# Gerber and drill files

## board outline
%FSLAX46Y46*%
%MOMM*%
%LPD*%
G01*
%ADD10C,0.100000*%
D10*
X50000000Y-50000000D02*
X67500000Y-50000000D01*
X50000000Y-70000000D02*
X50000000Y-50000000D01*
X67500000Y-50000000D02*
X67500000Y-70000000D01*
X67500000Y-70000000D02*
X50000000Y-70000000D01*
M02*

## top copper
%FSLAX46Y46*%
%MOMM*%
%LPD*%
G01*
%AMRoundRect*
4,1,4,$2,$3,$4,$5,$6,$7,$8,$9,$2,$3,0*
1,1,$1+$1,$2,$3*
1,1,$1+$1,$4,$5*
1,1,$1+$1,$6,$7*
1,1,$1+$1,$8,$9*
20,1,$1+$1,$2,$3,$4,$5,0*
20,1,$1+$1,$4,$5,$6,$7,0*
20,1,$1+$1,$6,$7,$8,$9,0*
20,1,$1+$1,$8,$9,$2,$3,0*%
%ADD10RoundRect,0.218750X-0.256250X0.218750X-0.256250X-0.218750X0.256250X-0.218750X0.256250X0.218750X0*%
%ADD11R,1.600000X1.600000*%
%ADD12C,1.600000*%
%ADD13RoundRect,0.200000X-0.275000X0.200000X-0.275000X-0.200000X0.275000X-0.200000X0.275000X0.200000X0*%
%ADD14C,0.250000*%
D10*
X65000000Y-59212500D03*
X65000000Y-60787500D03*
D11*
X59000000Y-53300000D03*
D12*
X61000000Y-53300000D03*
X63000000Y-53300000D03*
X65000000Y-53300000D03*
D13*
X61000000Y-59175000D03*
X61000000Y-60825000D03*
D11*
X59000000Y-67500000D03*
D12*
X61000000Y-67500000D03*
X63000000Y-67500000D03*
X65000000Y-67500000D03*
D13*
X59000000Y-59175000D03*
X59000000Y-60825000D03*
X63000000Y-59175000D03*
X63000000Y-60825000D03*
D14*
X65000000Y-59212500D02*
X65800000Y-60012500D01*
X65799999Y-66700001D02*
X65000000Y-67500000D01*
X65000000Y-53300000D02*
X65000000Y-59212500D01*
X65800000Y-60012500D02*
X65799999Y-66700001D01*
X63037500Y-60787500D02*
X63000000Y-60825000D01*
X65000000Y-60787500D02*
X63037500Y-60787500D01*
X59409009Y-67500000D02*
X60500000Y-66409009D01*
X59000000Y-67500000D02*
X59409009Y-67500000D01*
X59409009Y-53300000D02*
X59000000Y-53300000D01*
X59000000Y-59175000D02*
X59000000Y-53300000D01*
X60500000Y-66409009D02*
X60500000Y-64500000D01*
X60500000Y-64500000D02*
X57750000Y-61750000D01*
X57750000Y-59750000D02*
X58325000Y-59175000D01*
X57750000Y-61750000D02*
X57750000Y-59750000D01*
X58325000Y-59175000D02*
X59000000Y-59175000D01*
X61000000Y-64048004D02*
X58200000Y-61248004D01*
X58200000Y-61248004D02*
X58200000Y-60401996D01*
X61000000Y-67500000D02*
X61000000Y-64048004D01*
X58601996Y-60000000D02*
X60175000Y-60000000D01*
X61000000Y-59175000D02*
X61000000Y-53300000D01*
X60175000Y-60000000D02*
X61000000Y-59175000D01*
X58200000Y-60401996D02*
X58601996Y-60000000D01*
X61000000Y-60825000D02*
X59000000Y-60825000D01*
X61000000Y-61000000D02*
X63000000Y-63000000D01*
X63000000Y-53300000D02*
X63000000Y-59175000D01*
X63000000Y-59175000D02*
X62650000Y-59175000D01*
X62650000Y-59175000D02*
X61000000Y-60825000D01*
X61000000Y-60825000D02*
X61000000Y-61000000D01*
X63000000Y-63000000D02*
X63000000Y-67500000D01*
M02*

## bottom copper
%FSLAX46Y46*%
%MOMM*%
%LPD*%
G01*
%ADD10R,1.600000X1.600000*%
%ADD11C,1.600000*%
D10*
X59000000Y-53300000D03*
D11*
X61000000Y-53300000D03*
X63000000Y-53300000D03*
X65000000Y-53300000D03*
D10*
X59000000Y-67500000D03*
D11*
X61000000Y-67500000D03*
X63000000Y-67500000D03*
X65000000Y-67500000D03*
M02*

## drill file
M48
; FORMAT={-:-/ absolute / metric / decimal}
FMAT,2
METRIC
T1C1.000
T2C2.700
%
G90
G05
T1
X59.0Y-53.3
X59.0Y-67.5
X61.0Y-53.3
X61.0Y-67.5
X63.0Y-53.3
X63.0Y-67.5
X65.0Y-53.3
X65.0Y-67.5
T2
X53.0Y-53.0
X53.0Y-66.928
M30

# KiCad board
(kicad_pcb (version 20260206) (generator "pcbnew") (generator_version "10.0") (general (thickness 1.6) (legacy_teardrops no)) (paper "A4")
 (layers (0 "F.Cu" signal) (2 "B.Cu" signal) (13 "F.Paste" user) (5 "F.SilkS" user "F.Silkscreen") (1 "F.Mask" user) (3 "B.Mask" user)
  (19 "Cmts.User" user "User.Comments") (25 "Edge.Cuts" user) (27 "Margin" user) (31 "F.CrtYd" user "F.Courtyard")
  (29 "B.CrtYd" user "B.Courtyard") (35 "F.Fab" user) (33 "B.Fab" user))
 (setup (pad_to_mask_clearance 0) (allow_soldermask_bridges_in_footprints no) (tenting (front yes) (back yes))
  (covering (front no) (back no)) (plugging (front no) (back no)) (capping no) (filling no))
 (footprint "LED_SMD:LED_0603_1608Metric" (layer "F.Cu") (at 65 60 -90)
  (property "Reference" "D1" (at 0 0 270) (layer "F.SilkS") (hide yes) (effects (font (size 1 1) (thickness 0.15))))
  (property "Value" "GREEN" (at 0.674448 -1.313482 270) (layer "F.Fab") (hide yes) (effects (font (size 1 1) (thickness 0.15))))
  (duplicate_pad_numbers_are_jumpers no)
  (pad "1" smd roundrect (at -0.7875 0 270) (size 0.875 0.95) (layers "F.Cu" "F.Mask" "F.Paste") (roundrect_rratio 0.25) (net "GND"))
  (pad "2" smd roundrect (at 0.7875 0 270) (size 0.875 0.95) (layers "F.Cu" "F.Mask" "F.Paste") (roundrect_rratio 0.25) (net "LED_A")))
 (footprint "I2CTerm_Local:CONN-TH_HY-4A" (layer "F.Cu") (at 59 53.3 90)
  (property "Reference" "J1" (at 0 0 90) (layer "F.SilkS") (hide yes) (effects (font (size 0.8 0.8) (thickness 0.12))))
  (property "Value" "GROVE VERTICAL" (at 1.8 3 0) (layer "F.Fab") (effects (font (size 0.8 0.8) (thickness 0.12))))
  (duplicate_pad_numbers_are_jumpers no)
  (pad "1" thru_hole rect (at 0 0 90) (size 1.6 1.6) (drill 1) (layers "*.Cu" "*.Mask") (remove_unused_layers no) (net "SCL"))
  (pad "2" thru_hole circle (at 0 2 90) (size 1.6 1.6) (drill 1) (layers "*.Cu" "*.Mask") (remove_unused_layers no) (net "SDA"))
  (pad "3" thru_hole circle (at 0 4 90) (size 1.6 1.6) (drill 1) (layers "*.Cu" "*.Mask") (remove_unused_layers no) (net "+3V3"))
  (pad "4" thru_hole circle (at 0 6 90) (size 1.6 1.6) (drill 1) (layers "*.Cu" "*.Mask") (remove_unused_layers no) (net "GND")))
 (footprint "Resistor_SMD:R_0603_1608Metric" (layer "F.Cu") (at 61 60 -90)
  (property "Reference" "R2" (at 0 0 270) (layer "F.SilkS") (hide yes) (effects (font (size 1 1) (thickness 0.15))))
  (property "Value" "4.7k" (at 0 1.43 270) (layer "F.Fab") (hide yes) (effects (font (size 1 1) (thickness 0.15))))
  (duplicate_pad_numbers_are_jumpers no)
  (pad "1" smd roundrect (at -0.825 0 270) (size 0.8 0.95) (layers "F.Cu" "F.Mask" "F.Paste") (roundrect_rratio 0.25) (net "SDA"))
  (pad "2" smd roundrect (at 0.825 0 270) (size 0.8 0.95) (layers "F.Cu" "F.Mask" "F.Paste") (roundrect_rratio 0.25) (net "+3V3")))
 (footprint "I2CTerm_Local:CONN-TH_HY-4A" (layer "F.Cu") (at 59 67.5 90)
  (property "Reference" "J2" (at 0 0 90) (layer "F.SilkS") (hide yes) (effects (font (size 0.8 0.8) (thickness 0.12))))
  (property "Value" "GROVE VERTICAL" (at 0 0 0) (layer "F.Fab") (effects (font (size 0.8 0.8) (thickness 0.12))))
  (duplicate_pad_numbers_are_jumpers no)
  (pad "1" thru_hole rect (at 0 0 90) (size 1.6 1.6) (drill 1) (layers "*.Cu" "*.Mask") (remove_unused_layers no) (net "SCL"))
  (pad "2" thru_hole circle (at 0 2 90) (size 1.6 1.6) (drill 1) (layers "*.Cu" "*.Mask") (remove_unused_layers no) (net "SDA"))
  (pad "3" thru_hole circle (at 0 4 90) (size 1.6 1.6) (drill 1) (layers "*.Cu" "*.Mask") (remove_unused_layers no) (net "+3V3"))
  (pad "4" thru_hole circle (at 0 6 90) (size 1.6 1.6) (drill 1) (layers "*.Cu" "*.Mask") (remove_unused_layers no) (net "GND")))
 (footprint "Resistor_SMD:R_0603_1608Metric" (layer "F.Cu") (at 59 60 -90)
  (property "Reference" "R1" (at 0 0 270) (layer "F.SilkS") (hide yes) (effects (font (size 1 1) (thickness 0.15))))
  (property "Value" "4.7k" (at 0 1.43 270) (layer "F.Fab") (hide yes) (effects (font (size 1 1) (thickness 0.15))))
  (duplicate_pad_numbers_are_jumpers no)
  (pad "1" smd roundrect (at -0.825 0 270) (size 0.8 0.95) (layers "F.Cu" "F.Mask" "F.Paste") (roundrect_rratio 0.25) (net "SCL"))
  (pad "2" smd roundrect (at 0.825 0 270) (size 0.8 0.95) (layers "F.Cu" "F.Mask" "F.Paste") (roundrect_rratio 0.25) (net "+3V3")))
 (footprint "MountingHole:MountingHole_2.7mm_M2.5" (layer "F.Cu") (at 53 66.928487)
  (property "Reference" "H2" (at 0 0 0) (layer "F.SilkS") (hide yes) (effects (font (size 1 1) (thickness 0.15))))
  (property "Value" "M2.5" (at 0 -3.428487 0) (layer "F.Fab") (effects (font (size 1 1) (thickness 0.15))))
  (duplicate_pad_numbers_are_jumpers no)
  (pad "" np_thru_hole circle (at 0 0) (size 2.7 2.7) (drill 2.7) (layers "*.Cu" "*.Mask")))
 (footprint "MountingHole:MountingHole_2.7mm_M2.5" (layer "F.Cu") (at 53 53)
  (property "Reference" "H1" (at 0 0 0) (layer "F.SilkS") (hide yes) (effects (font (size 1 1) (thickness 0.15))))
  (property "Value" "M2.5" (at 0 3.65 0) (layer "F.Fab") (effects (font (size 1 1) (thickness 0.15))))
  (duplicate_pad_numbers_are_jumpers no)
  (pad "" np_thru_hole circle (at 0 0) (size 2.7 2.7) (drill 2.7) (layers "*.Cu" "*.Mask")))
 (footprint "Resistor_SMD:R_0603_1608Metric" (layer "F.Cu") (at 63 60 -90)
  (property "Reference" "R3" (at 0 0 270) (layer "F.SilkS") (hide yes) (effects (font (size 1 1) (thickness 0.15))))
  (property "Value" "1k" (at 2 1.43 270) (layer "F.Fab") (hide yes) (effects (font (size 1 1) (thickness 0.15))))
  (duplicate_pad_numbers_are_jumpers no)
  (pad "1" smd roundrect (at -0.825 0 270) (size 0.8 0.95) (layers "F.Cu" "F.Mask" "F.Paste") (roundrect_rratio 0.25) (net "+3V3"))
  (pad "2" smd roundrect (at 0.825 0 270) (size 0.8 0.95) (layers "F.Cu" "F.Mask" "F.Paste") (roundrect_rratio 0.25) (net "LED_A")))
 (gr_line (start 50 50) (end 67.5 50) (stroke (width 0.1) (type default)) (layer "Edge.Cuts"))
 (gr_line (start 50 70) (end 50 50) (stroke (width 0.1) (type default)) (layer "Edge.Cuts"))
 (gr_line (start 67.5 50) (end 67.5 70) (stroke (width 0.1) (type default)) (layer "Edge.Cuts"))
 (gr_line (start 67.5 70) (end 50 70) (stroke (width 0.1) (type default)) (layer "Edge.Cuts"))
 (segment (start 65 59.2125) (end 65.8 60.0125) (width 0.25) (layer "F.Cu") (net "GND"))
 (segment (start 65.799999 66.700001) (end 65 67.5) (width 0.25) (layer "F.Cu") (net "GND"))
 (segment (start 65 53.3) (end 65 59.2125) (width 0.25) (layer "F.Cu") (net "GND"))
 (segment (start 65.8 60.0125) (end 65.799999 66.700001) (width 0.25) (layer "F.Cu") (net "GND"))
 (segment (start 63.0375 60.7875) (end 63 60.825) (width 0.25) (layer "F.Cu") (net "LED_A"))
 (segment (start 65 60.7875) (end 63.0375 60.7875) (width 0.25) (layer "F.Cu") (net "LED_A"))
 (segment (start 59.409009 67.5) (end 60.5 66.409009) (width 0.25) (layer "F.Cu") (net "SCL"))
 (segment (start 59 67.5) (end 59.409009 67.5) (width 0.25) (layer "F.Cu") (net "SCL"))
 (segment (start 59.409009 53.3) (end 59 53.3) (width 0.25) (layer "F.Cu") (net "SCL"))
 (segment (start 59 59.175) (end 59 53.3) (width 0.25) (layer "F.Cu") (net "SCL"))
 (segment (start 60.5 66.409009) (end 60.5 64.5) (width 0.25) (layer "F.Cu") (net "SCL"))
 (segment (start 60.5 64.5) (end 57.75 61.75) (width 0.25) (layer "F.Cu") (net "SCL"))
 (segment (start 57.75 59.75) (end 58.325 59.175) (width 0.25) (layer "F.Cu") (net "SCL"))
 (segment (start 57.75 61.75) (end 57.75 59.75) (width 0.25) (layer "F.Cu") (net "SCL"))
 (segment (start 58.325 59.175) (end 59 59.175) (width 0.25) (layer "F.Cu") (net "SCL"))
 (segment (start 61 64.048004) (end 58.2 61.248004) (width 0.25) (layer "F.Cu") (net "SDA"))
 (segment (start 58.2 61.248004) (end 58.2 60.401996) (width 0.25) (layer "F.Cu") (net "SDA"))
 (segment (start 61 67.5) (end 61 64.048004) (width 0.25) (layer "F.Cu") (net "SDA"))
 (segment (start 58.601996 60) (end 60.175 60) (width 0.25) (layer "F.Cu") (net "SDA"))
 (segment (start 61 59.175) (end 61 53.3) (width 0.25) (layer "F.Cu") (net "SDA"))
 (segment (start 60.175 60) (end 61 59.175) (width 0.25) (layer "F.Cu") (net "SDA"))
 (segment (start 58.2 60.401996) (end 58.601996 60) (width 0.25) (layer "F.Cu") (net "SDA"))
 (segment (start 61 60.825) (end 59 60.825) (width 0.25) (layer "F.Cu") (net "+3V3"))
 (segment (start 61 61) (end 63 63) (width 0.25) (layer "F.Cu") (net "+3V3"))
 (segment (start 63 53.3) (end 63 59.175) (width 0.25) (layer "F.Cu") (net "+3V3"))
 (segment (start 63 59.175) (end 62.65 59.175) (width 0.25) (layer "F.Cu") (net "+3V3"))
 (segment (start 62.65 59.175) (end 61 60.825) (width 0.25) (layer "F.Cu") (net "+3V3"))
 (segment (start 61 60.825) (end 61 61) (width 0.25) (layer "F.Cu") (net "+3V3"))
 (segment (start 63 63) (end 63 67.5) (width 0.25) (layer "F.Cu") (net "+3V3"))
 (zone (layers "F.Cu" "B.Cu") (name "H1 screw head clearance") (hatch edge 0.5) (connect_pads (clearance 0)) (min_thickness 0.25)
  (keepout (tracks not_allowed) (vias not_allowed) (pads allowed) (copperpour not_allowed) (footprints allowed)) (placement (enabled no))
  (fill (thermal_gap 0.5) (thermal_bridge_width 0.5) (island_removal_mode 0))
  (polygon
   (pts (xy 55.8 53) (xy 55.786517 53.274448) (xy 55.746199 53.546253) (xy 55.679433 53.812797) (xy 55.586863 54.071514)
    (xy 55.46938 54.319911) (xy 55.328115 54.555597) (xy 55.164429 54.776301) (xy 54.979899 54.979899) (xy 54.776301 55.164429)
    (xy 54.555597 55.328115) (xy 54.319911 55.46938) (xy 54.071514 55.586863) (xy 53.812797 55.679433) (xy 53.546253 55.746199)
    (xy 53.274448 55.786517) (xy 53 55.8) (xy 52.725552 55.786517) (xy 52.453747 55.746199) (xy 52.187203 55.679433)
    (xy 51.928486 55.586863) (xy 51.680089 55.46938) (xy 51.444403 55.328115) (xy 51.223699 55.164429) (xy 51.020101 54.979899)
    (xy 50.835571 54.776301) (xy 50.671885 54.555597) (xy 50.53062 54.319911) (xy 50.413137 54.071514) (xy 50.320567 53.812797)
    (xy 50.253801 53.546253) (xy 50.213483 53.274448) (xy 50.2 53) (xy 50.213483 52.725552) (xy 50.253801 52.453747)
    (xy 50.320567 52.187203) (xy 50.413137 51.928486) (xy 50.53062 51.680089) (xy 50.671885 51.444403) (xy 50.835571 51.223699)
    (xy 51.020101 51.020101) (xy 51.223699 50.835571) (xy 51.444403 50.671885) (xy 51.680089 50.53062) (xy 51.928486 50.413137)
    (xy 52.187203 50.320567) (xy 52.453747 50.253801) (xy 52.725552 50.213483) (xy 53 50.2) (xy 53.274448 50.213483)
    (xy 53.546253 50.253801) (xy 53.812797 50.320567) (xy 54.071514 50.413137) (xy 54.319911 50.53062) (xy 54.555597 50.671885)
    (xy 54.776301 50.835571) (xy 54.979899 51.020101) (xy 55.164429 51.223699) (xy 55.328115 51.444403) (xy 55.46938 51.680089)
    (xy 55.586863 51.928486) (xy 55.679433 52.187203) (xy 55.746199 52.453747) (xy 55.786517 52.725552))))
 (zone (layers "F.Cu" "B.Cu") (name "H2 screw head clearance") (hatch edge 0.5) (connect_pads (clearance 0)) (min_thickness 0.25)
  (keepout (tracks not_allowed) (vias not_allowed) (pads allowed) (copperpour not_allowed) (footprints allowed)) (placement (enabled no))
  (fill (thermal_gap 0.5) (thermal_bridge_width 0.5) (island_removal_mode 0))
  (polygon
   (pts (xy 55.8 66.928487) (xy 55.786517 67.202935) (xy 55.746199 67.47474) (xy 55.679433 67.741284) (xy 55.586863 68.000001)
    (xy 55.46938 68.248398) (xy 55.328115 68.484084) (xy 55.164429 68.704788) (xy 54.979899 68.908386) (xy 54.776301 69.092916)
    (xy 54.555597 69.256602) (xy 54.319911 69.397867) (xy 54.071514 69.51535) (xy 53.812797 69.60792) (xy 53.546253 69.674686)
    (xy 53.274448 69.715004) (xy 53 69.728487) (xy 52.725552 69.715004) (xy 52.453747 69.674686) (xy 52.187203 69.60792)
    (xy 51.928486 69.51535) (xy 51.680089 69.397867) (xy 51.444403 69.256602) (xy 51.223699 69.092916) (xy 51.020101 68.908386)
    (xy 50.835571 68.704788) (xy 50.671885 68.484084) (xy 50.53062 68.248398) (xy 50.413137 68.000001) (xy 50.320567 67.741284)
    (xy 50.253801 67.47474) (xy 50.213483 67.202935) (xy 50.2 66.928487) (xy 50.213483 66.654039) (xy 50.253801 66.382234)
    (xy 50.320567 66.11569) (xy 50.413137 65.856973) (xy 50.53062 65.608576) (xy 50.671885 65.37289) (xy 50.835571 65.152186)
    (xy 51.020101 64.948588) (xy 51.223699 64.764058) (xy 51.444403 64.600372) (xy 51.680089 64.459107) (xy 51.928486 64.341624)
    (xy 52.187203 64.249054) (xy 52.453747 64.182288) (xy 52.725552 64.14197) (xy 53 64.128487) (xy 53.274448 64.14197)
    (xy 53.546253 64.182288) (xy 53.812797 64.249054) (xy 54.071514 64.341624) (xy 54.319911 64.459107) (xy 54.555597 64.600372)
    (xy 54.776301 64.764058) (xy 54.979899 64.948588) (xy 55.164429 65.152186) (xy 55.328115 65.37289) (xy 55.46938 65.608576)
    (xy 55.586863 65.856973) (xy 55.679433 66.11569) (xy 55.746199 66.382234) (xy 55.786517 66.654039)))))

